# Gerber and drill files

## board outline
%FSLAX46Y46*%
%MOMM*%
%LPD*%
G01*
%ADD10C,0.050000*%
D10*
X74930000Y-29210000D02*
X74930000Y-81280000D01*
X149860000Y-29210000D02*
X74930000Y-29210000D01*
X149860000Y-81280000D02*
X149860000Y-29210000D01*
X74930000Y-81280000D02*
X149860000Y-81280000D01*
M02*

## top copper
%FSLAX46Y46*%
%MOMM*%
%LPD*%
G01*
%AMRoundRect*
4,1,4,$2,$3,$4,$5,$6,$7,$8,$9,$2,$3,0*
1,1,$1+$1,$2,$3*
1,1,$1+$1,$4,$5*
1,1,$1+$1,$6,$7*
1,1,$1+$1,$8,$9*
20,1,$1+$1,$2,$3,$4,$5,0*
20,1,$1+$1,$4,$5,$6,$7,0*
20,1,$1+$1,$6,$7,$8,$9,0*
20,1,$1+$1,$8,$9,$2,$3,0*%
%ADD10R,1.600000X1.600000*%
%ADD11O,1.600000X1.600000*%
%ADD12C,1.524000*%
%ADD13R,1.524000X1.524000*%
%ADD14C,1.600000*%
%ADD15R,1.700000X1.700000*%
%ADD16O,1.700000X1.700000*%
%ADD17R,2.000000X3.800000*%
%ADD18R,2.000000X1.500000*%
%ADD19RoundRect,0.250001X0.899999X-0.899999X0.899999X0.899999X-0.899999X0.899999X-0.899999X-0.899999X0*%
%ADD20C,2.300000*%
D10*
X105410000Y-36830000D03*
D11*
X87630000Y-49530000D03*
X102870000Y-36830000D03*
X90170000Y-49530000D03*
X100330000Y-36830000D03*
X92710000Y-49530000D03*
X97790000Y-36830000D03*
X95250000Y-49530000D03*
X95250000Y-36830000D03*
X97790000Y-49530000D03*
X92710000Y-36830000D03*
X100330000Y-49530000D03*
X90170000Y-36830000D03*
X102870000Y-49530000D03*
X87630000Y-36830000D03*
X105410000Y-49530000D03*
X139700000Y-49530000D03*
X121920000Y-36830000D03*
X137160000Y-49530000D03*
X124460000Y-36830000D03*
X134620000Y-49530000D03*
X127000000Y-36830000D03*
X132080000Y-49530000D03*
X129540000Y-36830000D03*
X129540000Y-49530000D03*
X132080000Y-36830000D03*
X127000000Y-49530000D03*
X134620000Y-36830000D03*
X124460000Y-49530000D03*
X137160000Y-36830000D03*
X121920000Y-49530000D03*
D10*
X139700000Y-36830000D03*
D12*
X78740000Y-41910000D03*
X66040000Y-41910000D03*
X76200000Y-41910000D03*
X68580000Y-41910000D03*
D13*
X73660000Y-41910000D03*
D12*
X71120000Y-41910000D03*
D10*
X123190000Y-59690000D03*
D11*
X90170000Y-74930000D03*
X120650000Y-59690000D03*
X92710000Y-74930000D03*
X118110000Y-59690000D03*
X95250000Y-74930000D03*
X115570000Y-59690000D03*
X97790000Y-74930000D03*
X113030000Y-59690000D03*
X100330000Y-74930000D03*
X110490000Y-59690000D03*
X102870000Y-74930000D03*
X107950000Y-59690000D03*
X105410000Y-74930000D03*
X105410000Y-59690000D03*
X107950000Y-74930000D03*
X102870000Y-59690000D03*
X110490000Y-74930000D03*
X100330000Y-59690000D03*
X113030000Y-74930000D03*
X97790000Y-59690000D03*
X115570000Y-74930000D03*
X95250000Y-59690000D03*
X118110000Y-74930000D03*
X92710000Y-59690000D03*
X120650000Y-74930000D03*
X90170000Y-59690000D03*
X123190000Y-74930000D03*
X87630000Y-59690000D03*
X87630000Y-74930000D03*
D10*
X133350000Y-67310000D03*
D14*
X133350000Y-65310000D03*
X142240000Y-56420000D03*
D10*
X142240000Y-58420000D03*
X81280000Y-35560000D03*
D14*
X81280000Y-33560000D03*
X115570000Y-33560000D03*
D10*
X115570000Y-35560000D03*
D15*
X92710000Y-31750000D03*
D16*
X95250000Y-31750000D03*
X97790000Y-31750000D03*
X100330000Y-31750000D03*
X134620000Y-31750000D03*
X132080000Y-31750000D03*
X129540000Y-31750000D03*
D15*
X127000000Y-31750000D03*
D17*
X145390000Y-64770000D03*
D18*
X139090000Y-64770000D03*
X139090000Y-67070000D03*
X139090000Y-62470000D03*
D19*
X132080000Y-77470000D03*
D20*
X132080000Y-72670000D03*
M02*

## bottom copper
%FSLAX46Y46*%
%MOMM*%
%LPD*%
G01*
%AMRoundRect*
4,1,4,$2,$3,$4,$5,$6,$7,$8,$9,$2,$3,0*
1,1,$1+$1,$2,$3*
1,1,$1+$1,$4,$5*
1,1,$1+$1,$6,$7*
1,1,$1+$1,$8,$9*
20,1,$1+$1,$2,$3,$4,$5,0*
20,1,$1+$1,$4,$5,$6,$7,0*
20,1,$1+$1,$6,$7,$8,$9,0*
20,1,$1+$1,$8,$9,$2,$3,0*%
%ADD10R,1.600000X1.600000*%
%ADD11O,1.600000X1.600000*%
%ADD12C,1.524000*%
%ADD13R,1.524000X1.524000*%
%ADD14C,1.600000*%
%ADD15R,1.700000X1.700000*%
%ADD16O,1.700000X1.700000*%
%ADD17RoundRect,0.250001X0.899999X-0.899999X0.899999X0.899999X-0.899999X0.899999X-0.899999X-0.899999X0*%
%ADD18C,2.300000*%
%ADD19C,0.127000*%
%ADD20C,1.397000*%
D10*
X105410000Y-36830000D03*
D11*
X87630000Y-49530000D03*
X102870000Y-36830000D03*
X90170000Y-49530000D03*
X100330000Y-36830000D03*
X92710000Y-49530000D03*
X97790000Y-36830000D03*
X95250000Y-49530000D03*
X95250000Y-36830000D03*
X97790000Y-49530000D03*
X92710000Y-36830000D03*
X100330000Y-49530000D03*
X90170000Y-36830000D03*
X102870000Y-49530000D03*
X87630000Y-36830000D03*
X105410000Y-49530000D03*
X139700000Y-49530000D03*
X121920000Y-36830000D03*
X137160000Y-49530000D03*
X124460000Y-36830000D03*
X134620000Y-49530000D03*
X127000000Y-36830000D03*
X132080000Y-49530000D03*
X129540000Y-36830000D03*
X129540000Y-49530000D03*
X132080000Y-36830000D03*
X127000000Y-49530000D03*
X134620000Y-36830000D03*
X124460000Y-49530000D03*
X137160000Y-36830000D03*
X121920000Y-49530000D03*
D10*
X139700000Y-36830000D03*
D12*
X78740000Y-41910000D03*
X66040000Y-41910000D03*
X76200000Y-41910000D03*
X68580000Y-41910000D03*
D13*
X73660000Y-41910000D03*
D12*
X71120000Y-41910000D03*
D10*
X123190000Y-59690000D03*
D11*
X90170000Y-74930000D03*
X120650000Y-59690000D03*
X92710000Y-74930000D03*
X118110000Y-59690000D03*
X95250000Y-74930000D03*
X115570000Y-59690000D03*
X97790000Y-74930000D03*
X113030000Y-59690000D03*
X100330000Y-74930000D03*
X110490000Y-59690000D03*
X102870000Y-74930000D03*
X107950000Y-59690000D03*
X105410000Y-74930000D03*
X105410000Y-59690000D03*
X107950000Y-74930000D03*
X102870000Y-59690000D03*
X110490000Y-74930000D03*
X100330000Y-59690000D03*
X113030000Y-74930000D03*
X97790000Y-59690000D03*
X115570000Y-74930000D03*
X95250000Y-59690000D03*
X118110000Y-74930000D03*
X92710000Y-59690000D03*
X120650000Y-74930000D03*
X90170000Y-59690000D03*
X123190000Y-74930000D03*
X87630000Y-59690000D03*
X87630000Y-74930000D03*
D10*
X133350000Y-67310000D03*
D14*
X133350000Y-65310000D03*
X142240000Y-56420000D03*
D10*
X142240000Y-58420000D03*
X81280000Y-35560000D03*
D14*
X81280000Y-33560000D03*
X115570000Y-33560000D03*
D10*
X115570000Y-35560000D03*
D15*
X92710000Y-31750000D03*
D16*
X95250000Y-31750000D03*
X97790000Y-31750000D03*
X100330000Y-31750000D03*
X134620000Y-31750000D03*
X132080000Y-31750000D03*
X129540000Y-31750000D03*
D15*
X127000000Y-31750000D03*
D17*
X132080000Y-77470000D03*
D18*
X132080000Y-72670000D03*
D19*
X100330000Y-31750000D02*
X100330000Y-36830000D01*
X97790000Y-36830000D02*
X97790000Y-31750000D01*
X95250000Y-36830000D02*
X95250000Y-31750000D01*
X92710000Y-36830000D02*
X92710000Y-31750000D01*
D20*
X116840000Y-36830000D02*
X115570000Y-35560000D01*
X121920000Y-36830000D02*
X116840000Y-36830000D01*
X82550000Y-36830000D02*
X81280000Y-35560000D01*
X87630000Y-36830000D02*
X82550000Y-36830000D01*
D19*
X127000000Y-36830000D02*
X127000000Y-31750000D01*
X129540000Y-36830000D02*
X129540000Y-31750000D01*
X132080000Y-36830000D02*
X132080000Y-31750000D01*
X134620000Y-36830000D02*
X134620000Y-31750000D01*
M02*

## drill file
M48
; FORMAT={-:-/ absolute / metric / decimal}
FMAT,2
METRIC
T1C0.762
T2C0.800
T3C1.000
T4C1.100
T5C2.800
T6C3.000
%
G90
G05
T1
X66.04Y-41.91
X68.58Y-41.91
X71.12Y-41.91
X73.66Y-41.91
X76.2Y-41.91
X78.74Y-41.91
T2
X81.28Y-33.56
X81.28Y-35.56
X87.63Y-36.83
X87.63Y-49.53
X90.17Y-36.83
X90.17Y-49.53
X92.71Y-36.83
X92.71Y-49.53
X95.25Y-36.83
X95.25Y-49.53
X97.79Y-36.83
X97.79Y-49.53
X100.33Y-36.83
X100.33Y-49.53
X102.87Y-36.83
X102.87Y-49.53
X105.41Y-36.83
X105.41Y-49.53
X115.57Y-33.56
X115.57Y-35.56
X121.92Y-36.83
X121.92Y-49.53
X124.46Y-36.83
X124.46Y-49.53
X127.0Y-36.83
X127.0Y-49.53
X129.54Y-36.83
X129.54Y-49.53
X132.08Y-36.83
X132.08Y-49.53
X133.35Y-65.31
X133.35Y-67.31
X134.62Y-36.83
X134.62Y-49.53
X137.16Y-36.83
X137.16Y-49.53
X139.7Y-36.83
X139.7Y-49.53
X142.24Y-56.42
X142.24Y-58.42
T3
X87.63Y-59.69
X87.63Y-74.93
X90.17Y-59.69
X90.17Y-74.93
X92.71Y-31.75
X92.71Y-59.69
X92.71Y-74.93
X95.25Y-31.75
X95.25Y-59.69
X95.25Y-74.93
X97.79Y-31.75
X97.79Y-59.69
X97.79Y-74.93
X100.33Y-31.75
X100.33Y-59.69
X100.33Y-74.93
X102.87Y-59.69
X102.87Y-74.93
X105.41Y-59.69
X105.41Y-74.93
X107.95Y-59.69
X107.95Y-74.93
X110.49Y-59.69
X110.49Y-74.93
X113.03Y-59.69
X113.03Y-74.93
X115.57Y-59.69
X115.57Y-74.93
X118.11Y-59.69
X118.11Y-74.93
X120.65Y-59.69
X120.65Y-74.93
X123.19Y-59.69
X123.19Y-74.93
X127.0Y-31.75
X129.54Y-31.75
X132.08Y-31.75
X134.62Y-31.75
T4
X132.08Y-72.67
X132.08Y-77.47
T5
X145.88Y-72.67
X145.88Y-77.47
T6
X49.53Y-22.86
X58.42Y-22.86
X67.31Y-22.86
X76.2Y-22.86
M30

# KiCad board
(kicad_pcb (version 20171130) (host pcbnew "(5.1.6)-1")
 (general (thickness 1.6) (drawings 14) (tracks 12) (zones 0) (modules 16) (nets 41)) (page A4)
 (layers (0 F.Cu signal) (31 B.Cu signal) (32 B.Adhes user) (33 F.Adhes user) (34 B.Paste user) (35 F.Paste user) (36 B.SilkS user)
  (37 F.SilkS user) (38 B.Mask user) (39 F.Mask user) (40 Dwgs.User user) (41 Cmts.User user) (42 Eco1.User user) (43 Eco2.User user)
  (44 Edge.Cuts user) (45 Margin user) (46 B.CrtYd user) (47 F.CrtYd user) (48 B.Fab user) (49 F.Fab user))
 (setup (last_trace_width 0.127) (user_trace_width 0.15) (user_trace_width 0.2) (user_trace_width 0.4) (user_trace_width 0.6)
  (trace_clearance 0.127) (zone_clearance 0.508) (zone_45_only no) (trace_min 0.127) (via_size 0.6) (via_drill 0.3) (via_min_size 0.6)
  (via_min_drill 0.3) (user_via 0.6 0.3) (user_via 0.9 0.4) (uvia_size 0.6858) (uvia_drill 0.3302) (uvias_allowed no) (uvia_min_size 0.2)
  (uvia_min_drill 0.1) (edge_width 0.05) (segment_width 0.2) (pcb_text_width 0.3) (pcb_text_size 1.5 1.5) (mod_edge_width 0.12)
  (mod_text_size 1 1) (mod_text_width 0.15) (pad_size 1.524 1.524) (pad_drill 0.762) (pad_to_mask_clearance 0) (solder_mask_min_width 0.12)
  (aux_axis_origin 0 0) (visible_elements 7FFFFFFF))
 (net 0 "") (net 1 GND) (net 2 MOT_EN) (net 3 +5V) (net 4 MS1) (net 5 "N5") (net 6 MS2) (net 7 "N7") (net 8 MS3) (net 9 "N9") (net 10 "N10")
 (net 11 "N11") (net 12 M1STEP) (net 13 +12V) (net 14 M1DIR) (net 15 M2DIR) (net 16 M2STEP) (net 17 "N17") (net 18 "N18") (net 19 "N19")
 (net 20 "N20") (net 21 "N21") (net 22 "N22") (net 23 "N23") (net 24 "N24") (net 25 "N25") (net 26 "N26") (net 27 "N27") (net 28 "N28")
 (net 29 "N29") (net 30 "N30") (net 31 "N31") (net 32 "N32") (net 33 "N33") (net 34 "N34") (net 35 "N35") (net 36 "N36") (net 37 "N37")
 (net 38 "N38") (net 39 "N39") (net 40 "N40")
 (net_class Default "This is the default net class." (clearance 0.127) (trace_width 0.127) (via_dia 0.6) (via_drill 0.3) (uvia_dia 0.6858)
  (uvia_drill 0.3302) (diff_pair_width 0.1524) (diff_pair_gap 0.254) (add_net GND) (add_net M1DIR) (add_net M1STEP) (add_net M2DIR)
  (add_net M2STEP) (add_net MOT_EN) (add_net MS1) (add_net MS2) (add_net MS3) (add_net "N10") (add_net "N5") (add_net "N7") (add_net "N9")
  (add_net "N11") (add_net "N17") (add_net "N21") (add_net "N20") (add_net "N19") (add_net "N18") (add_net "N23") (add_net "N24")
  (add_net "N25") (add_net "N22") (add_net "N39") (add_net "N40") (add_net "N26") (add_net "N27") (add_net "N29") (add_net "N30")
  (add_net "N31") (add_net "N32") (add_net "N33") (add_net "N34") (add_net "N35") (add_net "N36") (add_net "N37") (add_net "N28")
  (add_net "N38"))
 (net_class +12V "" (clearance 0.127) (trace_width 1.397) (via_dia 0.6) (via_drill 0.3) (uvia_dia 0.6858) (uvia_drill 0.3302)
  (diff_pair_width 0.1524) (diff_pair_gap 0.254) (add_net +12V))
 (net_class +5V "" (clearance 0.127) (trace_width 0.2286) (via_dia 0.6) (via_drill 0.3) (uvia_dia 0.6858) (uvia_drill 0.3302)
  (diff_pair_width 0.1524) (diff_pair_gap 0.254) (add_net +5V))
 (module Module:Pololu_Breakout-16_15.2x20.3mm (layer F.Cu) (at 105.41 36.83 270)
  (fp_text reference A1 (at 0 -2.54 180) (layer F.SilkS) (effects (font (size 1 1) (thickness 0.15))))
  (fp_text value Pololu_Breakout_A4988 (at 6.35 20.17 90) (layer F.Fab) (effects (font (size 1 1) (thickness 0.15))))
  (pad 1 thru_hole rect (at 0 0 270) (size 1.6 1.6) (drill 0.8) (layers *.Cu *.Mask) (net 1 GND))
  (pad 9 thru_hole oval (at 12.7 17.78 270) (size 1.6 1.6) (drill 0.8) (layers *.Cu *.Mask) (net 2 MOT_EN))
  (pad 2 thru_hole oval (at 0 2.54 270) (size 1.6 1.6) (drill 0.8) (layers *.Cu *.Mask) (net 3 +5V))
  (pad 10 thru_hole oval (at 12.7 15.24 270) (size 1.6 1.6) (drill 0.8) (layers *.Cu *.Mask) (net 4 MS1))
  (pad 3 thru_hole oval (at 0 5.08 270) (size 1.6 1.6) (drill 0.8) (layers *.Cu *.Mask) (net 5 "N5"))
  (pad 11 thru_hole oval (at 12.7 12.7 270) (size 1.6 1.6) (drill 0.8) (layers *.Cu *.Mask) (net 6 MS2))
  (pad 4 thru_hole oval (at 0 7.62 270) (size 1.6 1.6) (drill 0.8) (layers *.Cu *.Mask) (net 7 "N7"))
  (pad 12 thru_hole oval (at 12.7 10.16 270) (size 1.6 1.6) (drill 0.8) (layers *.Cu *.Mask) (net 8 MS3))
  (pad 5 thru_hole oval (at 0 10.16 270) (size 1.6 1.6) (drill 0.8) (layers *.Cu *.Mask) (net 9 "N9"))
  (pad 13 thru_hole oval (at 12.7 7.62 270) (size 1.6 1.6) (drill 0.8) (layers *.Cu *.Mask) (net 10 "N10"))
  (pad 6 thru_hole oval (at 0 12.7 270) (size 1.6 1.6) (drill 0.8) (layers *.Cu *.Mask) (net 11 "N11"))
  (pad 14 thru_hole oval (at 12.7 5.08 270) (size 1.6 1.6) (drill 0.8) (layers *.Cu *.Mask) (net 10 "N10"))
  (pad 7 thru_hole oval (at 0 15.24 270) (size 1.6 1.6) (drill 0.8) (layers *.Cu *.Mask) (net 1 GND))
  (pad 15 thru_hole oval (at 12.7 2.54 270) (size 1.6 1.6) (drill 0.8) (layers *.Cu *.Mask) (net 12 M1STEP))
  (pad 8 thru_hole oval (at 0 17.78 270) (size 1.6 1.6) (drill 0.8) (layers *.Cu *.Mask) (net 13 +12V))
  (pad 16 thru_hole oval (at 12.7 0 270) (size 1.6 1.6) (drill 0.8) (layers *.Cu *.Mask) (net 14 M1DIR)))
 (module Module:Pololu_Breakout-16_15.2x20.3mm (layer F.Cu) (at 139.7 36.83 270)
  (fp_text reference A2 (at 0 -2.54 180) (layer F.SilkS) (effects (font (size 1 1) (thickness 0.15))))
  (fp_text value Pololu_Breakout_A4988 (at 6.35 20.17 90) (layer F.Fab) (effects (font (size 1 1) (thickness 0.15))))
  (pad 16 thru_hole oval (at 12.7 0 270) (size 1.6 1.6) (drill 0.8) (layers *.Cu *.Mask) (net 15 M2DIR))
  (pad 8 thru_hole oval (at 0 17.78 270) (size 1.6 1.6) (drill 0.8) (layers *.Cu *.Mask) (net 13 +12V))
  (pad 15 thru_hole oval (at 12.7 2.54 270) (size 1.6 1.6) (drill 0.8) (layers *.Cu *.Mask) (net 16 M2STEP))
  (pad 7 thru_hole oval (at 0 15.24 270) (size 1.6 1.6) (drill 0.8) (layers *.Cu *.Mask) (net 1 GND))
  (pad 14 thru_hole oval (at 12.7 5.08 270) (size 1.6 1.6) (drill 0.8) (layers *.Cu *.Mask) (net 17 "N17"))
  (pad 6 thru_hole oval (at 0 12.7 270) (size 1.6 1.6) (drill 0.8) (layers *.Cu *.Mask) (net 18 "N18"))
  (pad 13 thru_hole oval (at 12.7 7.62 270) (size 1.6 1.6) (drill 0.8) (layers *.Cu *.Mask) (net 17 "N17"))
  (pad 5 thru_hole oval (at 0 10.16 270) (size 1.6 1.6) (drill 0.8) (layers *.Cu *.Mask) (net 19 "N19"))
  (pad 12 thru_hole oval (at 12.7 10.16 270) (size 1.6 1.6) (drill 0.8) (layers *.Cu *.Mask) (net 8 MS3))
  (pad 4 thru_hole oval (at 0 7.62 270) (size 1.6 1.6) (drill 0.8) (layers *.Cu *.Mask) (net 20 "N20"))
  (pad 11 thru_hole oval (at 12.7 12.7 270) (size 1.6 1.6) (drill 0.8) (layers *.Cu *.Mask) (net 6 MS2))
  (pad 3 thru_hole oval (at 0 5.08 270) (size 1.6 1.6) (drill 0.8) (layers *.Cu *.Mask) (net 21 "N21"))
  (pad 10 thru_hole oval (at 12.7 15.24 270) (size 1.6 1.6) (drill 0.8) (layers *.Cu *.Mask) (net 4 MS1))
  (pad 2 thru_hole oval (at 0 2.54 270) (size 1.6 1.6) (drill 0.8) (layers *.Cu *.Mask) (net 3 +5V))
  (pad 9 thru_hole oval (at 12.7 17.78 270) (size 1.6 1.6) (drill 0.8) (layers *.Cu *.Mask) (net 2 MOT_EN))
  (pad 1 thru_hole rect (at 0 0 270) (size 1.6 1.6) (drill 0.8) (layers *.Cu *.Mask) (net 1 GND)))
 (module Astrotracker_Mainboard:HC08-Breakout (layer F.Cu) (at 72.39 41.91)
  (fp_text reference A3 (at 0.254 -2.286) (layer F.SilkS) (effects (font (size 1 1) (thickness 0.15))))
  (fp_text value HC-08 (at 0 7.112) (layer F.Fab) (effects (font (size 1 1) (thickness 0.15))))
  (pad 6 thru_hole circle (at 6.35 0) (size 1.524 1.524) (drill 0.762) (layers *.Cu *.Mask) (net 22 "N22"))
  (pad 1 thru_hole circle (at -6.35 0) (size 1.524 1.524) (drill 0.762) (layers *.Cu *.Mask) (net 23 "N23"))
  (pad 5 thru_hole circle (at 3.81 0) (size 1.524 1.524) (drill 0.762) (layers *.Cu *.Mask) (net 3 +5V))
  (pad 2 thru_hole circle (at -3.81 0) (size 1.524 1.524) (drill 0.762) (layers *.Cu *.Mask) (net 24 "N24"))
  (pad 4 thru_hole rect (at 1.27 0) (size 1.524 1.524) (drill 0.762) (layers *.Cu *.Mask) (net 1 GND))
  (pad 3 thru_hole circle (at -1.27 0) (size 1.524 1.524) (drill 0.762) (layers *.Cu *.Mask) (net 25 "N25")))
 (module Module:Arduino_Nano (layer F.Cu) (at 123.19 59.69 270)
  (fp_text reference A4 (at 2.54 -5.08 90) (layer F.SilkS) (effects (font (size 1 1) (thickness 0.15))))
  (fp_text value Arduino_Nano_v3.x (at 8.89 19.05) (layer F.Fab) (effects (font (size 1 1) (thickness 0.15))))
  (pad 1 thru_hole rect (at 0 0 270) (size 1.6 1.6) (drill 1) (layers *.Cu *.Mask) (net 24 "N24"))
  (pad 17 thru_hole oval (at 15.24 33.02 270) (size 1.6 1.6) (drill 1) (layers *.Cu *.Mask) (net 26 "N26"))
  (pad 2 thru_hole oval (at 0 2.54 270) (size 1.6 1.6) (drill 1) (layers *.Cu *.Mask) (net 25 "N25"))
  (pad 18 thru_hole oval (at 15.24 30.48 270) (size 1.6 1.6) (drill 1) (layers *.Cu *.Mask) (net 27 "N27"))
  (pad 3 thru_hole oval (at 0 5.08 270) (size 1.6 1.6) (drill 1) (layers *.Cu *.Mask) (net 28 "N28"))
  (pad 19 thru_hole oval (at 15.24 27.94 270) (size 1.6 1.6) (drill 1) (layers *.Cu *.Mask) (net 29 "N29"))
  (pad 4 thru_hole oval (at 0 7.62 270) (size 1.6 1.6) (drill 1) (layers *.Cu *.Mask) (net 1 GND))
  (pad 20 thru_hole oval (at 15.24 25.4 270) (size 1.6 1.6) (drill 1) (layers *.Cu *.Mask) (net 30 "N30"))
  (pad 5 thru_hole oval (at 0 10.16 270) (size 1.6 1.6) (drill 1) (layers *.Cu *.Mask) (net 23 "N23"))
  (pad 21 thru_hole oval (at 15.24 22.86 270) (size 1.6 1.6) (drill 1) (layers *.Cu *.Mask) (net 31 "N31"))
  (pad 6 thru_hole oval (at 0 12.7 270) (size 1.6 1.6) (drill 1) (layers *.Cu *.Mask) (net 22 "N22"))
  (pad 22 thru_hole oval (at 15.24 20.32 270) (size 1.6 1.6) (drill 1) (layers *.Cu *.Mask) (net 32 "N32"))
  (pad 7 thru_hole oval (at 0 15.24 270) (size 1.6 1.6) (drill 1) (layers *.Cu *.Mask) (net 12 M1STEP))
  (pad 23 thru_hole oval (at 15.24 17.78 270) (size 1.6 1.6) (drill 1) (layers *.Cu *.Mask) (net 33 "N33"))
  (pad 8 thru_hole oval (at 0 17.78 270) (size 1.6 1.6) (drill 1) (layers *.Cu *.Mask) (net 14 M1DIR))
  (pad 24 thru_hole oval (at 15.24 15.24 270) (size 1.6 1.6) (drill 1) (layers *.Cu *.Mask) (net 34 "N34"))
  (pad 9 thru_hole oval (at 0 20.32 270) (size 1.6 1.6) (drill 1) (layers *.Cu *.Mask) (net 16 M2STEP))
  (pad 25 thru_hole oval (at 15.24 12.7 270) (size 1.6 1.6) (drill 1) (layers *.Cu *.Mask) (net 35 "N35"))
  (pad 10 thru_hole oval (at 0 22.86 270) (size 1.6 1.6) (drill 1) (layers *.Cu *.Mask) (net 15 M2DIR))
  (pad 26 thru_hole oval (at 15.24 10.16 270) (size 1.6 1.6) (drill 1) (layers *.Cu *.Mask) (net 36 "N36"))
  (pad 11 thru_hole oval (at 0 25.4 270) (size 1.6 1.6) (drill 1) (layers *.Cu *.Mask) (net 2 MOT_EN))
  (pad 27 thru_hole oval (at 15.24 7.62 270) (size 1.6 1.6) (drill 1) (layers *.Cu *.Mask) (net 3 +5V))
  (pad 12 thru_hole oval (at 0 27.94 270) (size 1.6 1.6) (drill 1) (layers *.Cu *.Mask) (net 8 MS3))
  (pad 28 thru_hole oval (at 15.24 5.08 270) (size 1.6 1.6) (drill 1) (layers *.Cu *.Mask) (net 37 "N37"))
  (pad 13 thru_hole oval (at 0 30.48 270) (size 1.6 1.6) (drill 1) (layers *.Cu *.Mask) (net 6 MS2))
  (pad 29 thru_hole oval (at 15.24 2.54 270) (size 1.6 1.6) (drill 1) (layers *.Cu *.Mask) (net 1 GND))
  (pad 14 thru_hole oval (at 0 33.02 270) (size 1.6 1.6) (drill 1) (layers *.Cu *.Mask) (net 4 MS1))
  (pad 30 thru_hole oval (at 15.24 0 270) (size 1.6 1.6) (drill 1) (layers *.Cu *.Mask) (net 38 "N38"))
  (pad 15 thru_hole oval (at 0 35.56 270) (size 1.6 1.6) (drill 1) (layers *.Cu *.Mask) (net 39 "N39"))
  (pad 16 thru_hole oval (at 15.24 35.56 270) (size 1.6 1.6) (drill 1) (layers *.Cu *.Mask) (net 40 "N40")))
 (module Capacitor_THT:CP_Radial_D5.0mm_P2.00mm (layer F.Cu) (at 133.35 67.31 90)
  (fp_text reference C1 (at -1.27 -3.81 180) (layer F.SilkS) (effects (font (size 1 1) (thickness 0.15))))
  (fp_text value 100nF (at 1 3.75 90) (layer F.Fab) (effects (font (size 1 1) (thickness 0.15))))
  (pad 1 thru_hole rect (at 0 0 90) (size 1.6 1.6) (drill 0.8) (layers *.Cu *.Mask) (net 13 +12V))
  (pad 2 thru_hole circle (at 2 0 90) (size 1.6 1.6) (drill 0.8) (layers *.Cu *.Mask) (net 1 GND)))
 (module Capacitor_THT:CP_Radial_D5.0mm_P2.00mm (layer F.Cu) (at 142.24 58.42 90)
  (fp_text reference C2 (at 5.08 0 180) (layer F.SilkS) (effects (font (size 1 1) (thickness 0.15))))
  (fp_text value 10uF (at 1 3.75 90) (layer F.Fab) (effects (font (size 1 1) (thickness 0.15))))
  (pad 2 thru_hole circle (at 2 0 90) (size 1.6 1.6) (drill 0.8) (layers *.Cu *.Mask) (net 1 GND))
  (pad 1 thru_hole rect (at 0 0 90) (size 1.6 1.6) (drill 0.8) (layers *.Cu *.Mask) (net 3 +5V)))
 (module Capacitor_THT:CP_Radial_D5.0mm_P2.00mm (layer F.Cu) (at 81.28 35.56 90)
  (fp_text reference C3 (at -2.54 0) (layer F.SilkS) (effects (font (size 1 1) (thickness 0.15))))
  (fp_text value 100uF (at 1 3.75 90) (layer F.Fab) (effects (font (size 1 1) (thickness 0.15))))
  (pad 1 thru_hole rect (at 0 0 90) (size 1.6 1.6) (drill 0.8) (layers *.Cu *.Mask) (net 13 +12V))
  (pad 2 thru_hole circle (at 2 0 90) (size 1.6 1.6) (drill 0.8) (layers *.Cu *.Mask) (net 1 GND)))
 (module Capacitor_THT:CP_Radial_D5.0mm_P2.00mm (layer F.Cu) (at 115.57 35.56 90)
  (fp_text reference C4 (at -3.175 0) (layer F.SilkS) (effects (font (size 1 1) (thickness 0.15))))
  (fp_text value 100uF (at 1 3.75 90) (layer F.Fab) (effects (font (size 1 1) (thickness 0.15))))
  (pad 2 thru_hole circle (at 2 0 90) (size 1.6 1.6) (drill 0.8) (layers *.Cu *.Mask) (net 1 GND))
  (pad 1 thru_hole rect (at 0 0 90) (size 1.6 1.6) (drill 0.8) (layers *.Cu *.Mask) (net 13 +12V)))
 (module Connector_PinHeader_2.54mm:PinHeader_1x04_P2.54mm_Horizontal (layer F.Cu) (at 92.71 31.75 90)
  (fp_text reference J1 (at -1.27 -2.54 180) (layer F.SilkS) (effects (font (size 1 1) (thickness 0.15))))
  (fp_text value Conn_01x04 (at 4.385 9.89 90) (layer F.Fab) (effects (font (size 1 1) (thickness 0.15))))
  (pad 1 thru_hole rect (at 0 0 90) (size 1.7 1.7) (drill 1) (layers *.Cu *.Mask) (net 11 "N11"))
  (pad 2 thru_hole oval (at 0 2.54 90) (size 1.7 1.7) (drill 1) (layers *.Cu *.Mask) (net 9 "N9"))
  (pad 3 thru_hole oval (at 0 5.08 90) (size 1.7 1.7) (drill 1) (layers *.Cu *.Mask) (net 7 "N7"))
  (pad 4 thru_hole oval (at 0 7.62 90) (size 1.7 1.7) (drill 1) (layers *.Cu *.Mask) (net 5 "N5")))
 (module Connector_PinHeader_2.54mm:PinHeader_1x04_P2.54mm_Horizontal (layer F.Cu) (at 127 31.75 90)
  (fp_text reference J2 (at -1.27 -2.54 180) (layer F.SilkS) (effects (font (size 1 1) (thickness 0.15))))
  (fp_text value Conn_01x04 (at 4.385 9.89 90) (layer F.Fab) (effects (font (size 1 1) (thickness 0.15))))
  (pad 4 thru_hole oval (at 0 7.62 90) (size 1.7 1.7) (drill 1) (layers *.Cu *.Mask) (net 21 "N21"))
  (pad 3 thru_hole oval (at 0 5.08 90) (size 1.7 1.7) (drill 1) (layers *.Cu *.Mask) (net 20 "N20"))
  (pad 2 thru_hole oval (at 0 2.54 90) (size 1.7 1.7) (drill 1) (layers *.Cu *.Mask) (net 19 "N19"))
  (pad 1 thru_hole rect (at 0 0 90) (size 1.7 1.7) (drill 1) (layers *.Cu *.Mask) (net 18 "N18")))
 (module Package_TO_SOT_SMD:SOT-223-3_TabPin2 (layer F.Cu) (at 142.24 64.77)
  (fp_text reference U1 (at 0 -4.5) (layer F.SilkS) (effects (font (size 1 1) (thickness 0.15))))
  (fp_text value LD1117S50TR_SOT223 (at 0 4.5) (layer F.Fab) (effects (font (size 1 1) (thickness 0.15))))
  (pad 2 smd rect (at 3.15 0) (size 2 3.8) (layers F.Cu F.Paste F.Mask) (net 3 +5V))
  (pad 2 smd rect (at -3.15 0) (size 2 1.5) (layers F.Cu F.Paste F.Mask) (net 3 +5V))
  (pad 3 smd rect (at -3.15 2.3) (size 2 1.5) (layers F.Cu F.Paste F.Mask) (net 13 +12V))
  (pad 1 smd rect (at -3.15 -2.3) (size 2 1.5) (layers F.Cu F.Paste F.Mask) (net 1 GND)))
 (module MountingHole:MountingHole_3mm (layer F.Cu) (at 49.53 22.86)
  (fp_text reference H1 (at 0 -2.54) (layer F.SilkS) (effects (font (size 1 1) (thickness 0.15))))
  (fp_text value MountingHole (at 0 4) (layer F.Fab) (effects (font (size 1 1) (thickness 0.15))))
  (pad 1 np_thru_hole circle (at 0 0) (size 3 3) (drill 3) (layers *.Cu *.Mask)))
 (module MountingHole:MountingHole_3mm (layer F.Cu) (at 58.42 22.86)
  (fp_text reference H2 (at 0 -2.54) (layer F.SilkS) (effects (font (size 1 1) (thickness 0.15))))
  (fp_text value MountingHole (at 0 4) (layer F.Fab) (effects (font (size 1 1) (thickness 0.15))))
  (pad 1 np_thru_hole circle (at 0 0) (size 3 3) (drill 3) (layers *.Cu *.Mask)))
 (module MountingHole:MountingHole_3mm (layer F.Cu) (at 67.31 22.86)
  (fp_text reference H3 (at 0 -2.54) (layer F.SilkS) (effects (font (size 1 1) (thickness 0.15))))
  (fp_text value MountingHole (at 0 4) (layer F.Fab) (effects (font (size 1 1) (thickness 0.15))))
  (pad 1 np_thru_hole circle (at 0 0) (size 3 3) (drill 3) (layers *.Cu *.Mask)))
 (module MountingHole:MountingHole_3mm (layer F.Cu) (at 76.2 22.86)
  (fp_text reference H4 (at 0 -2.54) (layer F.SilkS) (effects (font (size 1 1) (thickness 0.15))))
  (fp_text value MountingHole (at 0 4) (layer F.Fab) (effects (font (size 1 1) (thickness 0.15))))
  (pad 1 np_thru_hole circle (at 0 0) (size 3 3) (drill 3) (layers *.Cu *.Mask)))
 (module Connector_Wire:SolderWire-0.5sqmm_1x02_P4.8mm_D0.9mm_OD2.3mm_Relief (layer F.Cu) (at 132.08 77.47 90)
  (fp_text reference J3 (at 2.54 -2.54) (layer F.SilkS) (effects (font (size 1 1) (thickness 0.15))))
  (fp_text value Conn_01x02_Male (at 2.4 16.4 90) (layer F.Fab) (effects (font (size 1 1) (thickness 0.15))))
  (pad 1 thru_hole roundrect (at 0 0 90) (size 2.3 2.3) (drill 1.1) (layers *.Cu *.Mask) (roundrect_rratio 0.108696) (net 1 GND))
  (pad 2 thru_hole circle (at 4.8 0 90) (size 2.3 2.3) (drill 1.1) (layers *.Cu *.Mask) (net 13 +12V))
  (pad "" np_thru_hole circle (at 0 13.8 90) (size 2.8 2.8) (drill 2.8) (layers *.Cu *.Mask))
  (pad "" np_thru_hole circle (at 4.8 13.8 90) (size 2.8 2.8) (drill 2.8) (layers *.Cu *.Mask)))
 (gr_line (start 74.93 29.21) (end 74.93 81.28) (layer Edge.Cuts) (width 0.05))
 (gr_line (start 149.86 29.21) (end 74.93 29.21) (layer Edge.Cuts) (width 0.05))
 (gr_line (start 149.86 81.28) (end 149.86 29.21) (layer Edge.Cuts) (width 0.05))
 (gr_line (start 74.93 81.28) (end 149.86 81.28) (layer Edge.Cuts) (width 0.05))
 (segment (start 100.33 31.75) (end 100.33 36.83) (width 0.127) (layer B.Cu) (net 5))
 (segment (start 97.79 36.83) (end 97.79 31.75) (width 0.127) (layer B.Cu) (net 7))
 (segment (start 95.25 36.83) (end 95.25 31.75) (width 0.127) (layer B.Cu) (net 9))
 (segment (start 92.71 36.83) (end 92.71 31.75) (width 0.127) (layer B.Cu) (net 11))
 (segment (start 116.84 36.83) (end 115.57 35.56) (width 1.397) (layer B.Cu) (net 13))
 (segment (start 121.92 36.83) (end 116.84 36.83) (width 1.397) (layer B.Cu) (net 13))
 (segment (start 82.55 36.83) (end 81.28 35.56) (width 1.397) (layer B.Cu) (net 13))
 (segment (start 87.63 36.83) (end 82.55 36.83) (width 1.397) (layer B.Cu) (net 13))
 (segment (start 127 36.83) (end 127 31.75) (width 0.127) (layer B.Cu) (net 18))
 (segment (start 129.54 36.83) (end 129.54 31.75) (width 0.127) (layer B.Cu) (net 19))
 (segment (start 132.08 36.83) (end 132.08 31.75) (width 0.127) (layer B.Cu) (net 20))
 (segment (start 134.62 36.83) (end 134.62 31.75) (width 0.127) (layer B.Cu) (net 21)))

